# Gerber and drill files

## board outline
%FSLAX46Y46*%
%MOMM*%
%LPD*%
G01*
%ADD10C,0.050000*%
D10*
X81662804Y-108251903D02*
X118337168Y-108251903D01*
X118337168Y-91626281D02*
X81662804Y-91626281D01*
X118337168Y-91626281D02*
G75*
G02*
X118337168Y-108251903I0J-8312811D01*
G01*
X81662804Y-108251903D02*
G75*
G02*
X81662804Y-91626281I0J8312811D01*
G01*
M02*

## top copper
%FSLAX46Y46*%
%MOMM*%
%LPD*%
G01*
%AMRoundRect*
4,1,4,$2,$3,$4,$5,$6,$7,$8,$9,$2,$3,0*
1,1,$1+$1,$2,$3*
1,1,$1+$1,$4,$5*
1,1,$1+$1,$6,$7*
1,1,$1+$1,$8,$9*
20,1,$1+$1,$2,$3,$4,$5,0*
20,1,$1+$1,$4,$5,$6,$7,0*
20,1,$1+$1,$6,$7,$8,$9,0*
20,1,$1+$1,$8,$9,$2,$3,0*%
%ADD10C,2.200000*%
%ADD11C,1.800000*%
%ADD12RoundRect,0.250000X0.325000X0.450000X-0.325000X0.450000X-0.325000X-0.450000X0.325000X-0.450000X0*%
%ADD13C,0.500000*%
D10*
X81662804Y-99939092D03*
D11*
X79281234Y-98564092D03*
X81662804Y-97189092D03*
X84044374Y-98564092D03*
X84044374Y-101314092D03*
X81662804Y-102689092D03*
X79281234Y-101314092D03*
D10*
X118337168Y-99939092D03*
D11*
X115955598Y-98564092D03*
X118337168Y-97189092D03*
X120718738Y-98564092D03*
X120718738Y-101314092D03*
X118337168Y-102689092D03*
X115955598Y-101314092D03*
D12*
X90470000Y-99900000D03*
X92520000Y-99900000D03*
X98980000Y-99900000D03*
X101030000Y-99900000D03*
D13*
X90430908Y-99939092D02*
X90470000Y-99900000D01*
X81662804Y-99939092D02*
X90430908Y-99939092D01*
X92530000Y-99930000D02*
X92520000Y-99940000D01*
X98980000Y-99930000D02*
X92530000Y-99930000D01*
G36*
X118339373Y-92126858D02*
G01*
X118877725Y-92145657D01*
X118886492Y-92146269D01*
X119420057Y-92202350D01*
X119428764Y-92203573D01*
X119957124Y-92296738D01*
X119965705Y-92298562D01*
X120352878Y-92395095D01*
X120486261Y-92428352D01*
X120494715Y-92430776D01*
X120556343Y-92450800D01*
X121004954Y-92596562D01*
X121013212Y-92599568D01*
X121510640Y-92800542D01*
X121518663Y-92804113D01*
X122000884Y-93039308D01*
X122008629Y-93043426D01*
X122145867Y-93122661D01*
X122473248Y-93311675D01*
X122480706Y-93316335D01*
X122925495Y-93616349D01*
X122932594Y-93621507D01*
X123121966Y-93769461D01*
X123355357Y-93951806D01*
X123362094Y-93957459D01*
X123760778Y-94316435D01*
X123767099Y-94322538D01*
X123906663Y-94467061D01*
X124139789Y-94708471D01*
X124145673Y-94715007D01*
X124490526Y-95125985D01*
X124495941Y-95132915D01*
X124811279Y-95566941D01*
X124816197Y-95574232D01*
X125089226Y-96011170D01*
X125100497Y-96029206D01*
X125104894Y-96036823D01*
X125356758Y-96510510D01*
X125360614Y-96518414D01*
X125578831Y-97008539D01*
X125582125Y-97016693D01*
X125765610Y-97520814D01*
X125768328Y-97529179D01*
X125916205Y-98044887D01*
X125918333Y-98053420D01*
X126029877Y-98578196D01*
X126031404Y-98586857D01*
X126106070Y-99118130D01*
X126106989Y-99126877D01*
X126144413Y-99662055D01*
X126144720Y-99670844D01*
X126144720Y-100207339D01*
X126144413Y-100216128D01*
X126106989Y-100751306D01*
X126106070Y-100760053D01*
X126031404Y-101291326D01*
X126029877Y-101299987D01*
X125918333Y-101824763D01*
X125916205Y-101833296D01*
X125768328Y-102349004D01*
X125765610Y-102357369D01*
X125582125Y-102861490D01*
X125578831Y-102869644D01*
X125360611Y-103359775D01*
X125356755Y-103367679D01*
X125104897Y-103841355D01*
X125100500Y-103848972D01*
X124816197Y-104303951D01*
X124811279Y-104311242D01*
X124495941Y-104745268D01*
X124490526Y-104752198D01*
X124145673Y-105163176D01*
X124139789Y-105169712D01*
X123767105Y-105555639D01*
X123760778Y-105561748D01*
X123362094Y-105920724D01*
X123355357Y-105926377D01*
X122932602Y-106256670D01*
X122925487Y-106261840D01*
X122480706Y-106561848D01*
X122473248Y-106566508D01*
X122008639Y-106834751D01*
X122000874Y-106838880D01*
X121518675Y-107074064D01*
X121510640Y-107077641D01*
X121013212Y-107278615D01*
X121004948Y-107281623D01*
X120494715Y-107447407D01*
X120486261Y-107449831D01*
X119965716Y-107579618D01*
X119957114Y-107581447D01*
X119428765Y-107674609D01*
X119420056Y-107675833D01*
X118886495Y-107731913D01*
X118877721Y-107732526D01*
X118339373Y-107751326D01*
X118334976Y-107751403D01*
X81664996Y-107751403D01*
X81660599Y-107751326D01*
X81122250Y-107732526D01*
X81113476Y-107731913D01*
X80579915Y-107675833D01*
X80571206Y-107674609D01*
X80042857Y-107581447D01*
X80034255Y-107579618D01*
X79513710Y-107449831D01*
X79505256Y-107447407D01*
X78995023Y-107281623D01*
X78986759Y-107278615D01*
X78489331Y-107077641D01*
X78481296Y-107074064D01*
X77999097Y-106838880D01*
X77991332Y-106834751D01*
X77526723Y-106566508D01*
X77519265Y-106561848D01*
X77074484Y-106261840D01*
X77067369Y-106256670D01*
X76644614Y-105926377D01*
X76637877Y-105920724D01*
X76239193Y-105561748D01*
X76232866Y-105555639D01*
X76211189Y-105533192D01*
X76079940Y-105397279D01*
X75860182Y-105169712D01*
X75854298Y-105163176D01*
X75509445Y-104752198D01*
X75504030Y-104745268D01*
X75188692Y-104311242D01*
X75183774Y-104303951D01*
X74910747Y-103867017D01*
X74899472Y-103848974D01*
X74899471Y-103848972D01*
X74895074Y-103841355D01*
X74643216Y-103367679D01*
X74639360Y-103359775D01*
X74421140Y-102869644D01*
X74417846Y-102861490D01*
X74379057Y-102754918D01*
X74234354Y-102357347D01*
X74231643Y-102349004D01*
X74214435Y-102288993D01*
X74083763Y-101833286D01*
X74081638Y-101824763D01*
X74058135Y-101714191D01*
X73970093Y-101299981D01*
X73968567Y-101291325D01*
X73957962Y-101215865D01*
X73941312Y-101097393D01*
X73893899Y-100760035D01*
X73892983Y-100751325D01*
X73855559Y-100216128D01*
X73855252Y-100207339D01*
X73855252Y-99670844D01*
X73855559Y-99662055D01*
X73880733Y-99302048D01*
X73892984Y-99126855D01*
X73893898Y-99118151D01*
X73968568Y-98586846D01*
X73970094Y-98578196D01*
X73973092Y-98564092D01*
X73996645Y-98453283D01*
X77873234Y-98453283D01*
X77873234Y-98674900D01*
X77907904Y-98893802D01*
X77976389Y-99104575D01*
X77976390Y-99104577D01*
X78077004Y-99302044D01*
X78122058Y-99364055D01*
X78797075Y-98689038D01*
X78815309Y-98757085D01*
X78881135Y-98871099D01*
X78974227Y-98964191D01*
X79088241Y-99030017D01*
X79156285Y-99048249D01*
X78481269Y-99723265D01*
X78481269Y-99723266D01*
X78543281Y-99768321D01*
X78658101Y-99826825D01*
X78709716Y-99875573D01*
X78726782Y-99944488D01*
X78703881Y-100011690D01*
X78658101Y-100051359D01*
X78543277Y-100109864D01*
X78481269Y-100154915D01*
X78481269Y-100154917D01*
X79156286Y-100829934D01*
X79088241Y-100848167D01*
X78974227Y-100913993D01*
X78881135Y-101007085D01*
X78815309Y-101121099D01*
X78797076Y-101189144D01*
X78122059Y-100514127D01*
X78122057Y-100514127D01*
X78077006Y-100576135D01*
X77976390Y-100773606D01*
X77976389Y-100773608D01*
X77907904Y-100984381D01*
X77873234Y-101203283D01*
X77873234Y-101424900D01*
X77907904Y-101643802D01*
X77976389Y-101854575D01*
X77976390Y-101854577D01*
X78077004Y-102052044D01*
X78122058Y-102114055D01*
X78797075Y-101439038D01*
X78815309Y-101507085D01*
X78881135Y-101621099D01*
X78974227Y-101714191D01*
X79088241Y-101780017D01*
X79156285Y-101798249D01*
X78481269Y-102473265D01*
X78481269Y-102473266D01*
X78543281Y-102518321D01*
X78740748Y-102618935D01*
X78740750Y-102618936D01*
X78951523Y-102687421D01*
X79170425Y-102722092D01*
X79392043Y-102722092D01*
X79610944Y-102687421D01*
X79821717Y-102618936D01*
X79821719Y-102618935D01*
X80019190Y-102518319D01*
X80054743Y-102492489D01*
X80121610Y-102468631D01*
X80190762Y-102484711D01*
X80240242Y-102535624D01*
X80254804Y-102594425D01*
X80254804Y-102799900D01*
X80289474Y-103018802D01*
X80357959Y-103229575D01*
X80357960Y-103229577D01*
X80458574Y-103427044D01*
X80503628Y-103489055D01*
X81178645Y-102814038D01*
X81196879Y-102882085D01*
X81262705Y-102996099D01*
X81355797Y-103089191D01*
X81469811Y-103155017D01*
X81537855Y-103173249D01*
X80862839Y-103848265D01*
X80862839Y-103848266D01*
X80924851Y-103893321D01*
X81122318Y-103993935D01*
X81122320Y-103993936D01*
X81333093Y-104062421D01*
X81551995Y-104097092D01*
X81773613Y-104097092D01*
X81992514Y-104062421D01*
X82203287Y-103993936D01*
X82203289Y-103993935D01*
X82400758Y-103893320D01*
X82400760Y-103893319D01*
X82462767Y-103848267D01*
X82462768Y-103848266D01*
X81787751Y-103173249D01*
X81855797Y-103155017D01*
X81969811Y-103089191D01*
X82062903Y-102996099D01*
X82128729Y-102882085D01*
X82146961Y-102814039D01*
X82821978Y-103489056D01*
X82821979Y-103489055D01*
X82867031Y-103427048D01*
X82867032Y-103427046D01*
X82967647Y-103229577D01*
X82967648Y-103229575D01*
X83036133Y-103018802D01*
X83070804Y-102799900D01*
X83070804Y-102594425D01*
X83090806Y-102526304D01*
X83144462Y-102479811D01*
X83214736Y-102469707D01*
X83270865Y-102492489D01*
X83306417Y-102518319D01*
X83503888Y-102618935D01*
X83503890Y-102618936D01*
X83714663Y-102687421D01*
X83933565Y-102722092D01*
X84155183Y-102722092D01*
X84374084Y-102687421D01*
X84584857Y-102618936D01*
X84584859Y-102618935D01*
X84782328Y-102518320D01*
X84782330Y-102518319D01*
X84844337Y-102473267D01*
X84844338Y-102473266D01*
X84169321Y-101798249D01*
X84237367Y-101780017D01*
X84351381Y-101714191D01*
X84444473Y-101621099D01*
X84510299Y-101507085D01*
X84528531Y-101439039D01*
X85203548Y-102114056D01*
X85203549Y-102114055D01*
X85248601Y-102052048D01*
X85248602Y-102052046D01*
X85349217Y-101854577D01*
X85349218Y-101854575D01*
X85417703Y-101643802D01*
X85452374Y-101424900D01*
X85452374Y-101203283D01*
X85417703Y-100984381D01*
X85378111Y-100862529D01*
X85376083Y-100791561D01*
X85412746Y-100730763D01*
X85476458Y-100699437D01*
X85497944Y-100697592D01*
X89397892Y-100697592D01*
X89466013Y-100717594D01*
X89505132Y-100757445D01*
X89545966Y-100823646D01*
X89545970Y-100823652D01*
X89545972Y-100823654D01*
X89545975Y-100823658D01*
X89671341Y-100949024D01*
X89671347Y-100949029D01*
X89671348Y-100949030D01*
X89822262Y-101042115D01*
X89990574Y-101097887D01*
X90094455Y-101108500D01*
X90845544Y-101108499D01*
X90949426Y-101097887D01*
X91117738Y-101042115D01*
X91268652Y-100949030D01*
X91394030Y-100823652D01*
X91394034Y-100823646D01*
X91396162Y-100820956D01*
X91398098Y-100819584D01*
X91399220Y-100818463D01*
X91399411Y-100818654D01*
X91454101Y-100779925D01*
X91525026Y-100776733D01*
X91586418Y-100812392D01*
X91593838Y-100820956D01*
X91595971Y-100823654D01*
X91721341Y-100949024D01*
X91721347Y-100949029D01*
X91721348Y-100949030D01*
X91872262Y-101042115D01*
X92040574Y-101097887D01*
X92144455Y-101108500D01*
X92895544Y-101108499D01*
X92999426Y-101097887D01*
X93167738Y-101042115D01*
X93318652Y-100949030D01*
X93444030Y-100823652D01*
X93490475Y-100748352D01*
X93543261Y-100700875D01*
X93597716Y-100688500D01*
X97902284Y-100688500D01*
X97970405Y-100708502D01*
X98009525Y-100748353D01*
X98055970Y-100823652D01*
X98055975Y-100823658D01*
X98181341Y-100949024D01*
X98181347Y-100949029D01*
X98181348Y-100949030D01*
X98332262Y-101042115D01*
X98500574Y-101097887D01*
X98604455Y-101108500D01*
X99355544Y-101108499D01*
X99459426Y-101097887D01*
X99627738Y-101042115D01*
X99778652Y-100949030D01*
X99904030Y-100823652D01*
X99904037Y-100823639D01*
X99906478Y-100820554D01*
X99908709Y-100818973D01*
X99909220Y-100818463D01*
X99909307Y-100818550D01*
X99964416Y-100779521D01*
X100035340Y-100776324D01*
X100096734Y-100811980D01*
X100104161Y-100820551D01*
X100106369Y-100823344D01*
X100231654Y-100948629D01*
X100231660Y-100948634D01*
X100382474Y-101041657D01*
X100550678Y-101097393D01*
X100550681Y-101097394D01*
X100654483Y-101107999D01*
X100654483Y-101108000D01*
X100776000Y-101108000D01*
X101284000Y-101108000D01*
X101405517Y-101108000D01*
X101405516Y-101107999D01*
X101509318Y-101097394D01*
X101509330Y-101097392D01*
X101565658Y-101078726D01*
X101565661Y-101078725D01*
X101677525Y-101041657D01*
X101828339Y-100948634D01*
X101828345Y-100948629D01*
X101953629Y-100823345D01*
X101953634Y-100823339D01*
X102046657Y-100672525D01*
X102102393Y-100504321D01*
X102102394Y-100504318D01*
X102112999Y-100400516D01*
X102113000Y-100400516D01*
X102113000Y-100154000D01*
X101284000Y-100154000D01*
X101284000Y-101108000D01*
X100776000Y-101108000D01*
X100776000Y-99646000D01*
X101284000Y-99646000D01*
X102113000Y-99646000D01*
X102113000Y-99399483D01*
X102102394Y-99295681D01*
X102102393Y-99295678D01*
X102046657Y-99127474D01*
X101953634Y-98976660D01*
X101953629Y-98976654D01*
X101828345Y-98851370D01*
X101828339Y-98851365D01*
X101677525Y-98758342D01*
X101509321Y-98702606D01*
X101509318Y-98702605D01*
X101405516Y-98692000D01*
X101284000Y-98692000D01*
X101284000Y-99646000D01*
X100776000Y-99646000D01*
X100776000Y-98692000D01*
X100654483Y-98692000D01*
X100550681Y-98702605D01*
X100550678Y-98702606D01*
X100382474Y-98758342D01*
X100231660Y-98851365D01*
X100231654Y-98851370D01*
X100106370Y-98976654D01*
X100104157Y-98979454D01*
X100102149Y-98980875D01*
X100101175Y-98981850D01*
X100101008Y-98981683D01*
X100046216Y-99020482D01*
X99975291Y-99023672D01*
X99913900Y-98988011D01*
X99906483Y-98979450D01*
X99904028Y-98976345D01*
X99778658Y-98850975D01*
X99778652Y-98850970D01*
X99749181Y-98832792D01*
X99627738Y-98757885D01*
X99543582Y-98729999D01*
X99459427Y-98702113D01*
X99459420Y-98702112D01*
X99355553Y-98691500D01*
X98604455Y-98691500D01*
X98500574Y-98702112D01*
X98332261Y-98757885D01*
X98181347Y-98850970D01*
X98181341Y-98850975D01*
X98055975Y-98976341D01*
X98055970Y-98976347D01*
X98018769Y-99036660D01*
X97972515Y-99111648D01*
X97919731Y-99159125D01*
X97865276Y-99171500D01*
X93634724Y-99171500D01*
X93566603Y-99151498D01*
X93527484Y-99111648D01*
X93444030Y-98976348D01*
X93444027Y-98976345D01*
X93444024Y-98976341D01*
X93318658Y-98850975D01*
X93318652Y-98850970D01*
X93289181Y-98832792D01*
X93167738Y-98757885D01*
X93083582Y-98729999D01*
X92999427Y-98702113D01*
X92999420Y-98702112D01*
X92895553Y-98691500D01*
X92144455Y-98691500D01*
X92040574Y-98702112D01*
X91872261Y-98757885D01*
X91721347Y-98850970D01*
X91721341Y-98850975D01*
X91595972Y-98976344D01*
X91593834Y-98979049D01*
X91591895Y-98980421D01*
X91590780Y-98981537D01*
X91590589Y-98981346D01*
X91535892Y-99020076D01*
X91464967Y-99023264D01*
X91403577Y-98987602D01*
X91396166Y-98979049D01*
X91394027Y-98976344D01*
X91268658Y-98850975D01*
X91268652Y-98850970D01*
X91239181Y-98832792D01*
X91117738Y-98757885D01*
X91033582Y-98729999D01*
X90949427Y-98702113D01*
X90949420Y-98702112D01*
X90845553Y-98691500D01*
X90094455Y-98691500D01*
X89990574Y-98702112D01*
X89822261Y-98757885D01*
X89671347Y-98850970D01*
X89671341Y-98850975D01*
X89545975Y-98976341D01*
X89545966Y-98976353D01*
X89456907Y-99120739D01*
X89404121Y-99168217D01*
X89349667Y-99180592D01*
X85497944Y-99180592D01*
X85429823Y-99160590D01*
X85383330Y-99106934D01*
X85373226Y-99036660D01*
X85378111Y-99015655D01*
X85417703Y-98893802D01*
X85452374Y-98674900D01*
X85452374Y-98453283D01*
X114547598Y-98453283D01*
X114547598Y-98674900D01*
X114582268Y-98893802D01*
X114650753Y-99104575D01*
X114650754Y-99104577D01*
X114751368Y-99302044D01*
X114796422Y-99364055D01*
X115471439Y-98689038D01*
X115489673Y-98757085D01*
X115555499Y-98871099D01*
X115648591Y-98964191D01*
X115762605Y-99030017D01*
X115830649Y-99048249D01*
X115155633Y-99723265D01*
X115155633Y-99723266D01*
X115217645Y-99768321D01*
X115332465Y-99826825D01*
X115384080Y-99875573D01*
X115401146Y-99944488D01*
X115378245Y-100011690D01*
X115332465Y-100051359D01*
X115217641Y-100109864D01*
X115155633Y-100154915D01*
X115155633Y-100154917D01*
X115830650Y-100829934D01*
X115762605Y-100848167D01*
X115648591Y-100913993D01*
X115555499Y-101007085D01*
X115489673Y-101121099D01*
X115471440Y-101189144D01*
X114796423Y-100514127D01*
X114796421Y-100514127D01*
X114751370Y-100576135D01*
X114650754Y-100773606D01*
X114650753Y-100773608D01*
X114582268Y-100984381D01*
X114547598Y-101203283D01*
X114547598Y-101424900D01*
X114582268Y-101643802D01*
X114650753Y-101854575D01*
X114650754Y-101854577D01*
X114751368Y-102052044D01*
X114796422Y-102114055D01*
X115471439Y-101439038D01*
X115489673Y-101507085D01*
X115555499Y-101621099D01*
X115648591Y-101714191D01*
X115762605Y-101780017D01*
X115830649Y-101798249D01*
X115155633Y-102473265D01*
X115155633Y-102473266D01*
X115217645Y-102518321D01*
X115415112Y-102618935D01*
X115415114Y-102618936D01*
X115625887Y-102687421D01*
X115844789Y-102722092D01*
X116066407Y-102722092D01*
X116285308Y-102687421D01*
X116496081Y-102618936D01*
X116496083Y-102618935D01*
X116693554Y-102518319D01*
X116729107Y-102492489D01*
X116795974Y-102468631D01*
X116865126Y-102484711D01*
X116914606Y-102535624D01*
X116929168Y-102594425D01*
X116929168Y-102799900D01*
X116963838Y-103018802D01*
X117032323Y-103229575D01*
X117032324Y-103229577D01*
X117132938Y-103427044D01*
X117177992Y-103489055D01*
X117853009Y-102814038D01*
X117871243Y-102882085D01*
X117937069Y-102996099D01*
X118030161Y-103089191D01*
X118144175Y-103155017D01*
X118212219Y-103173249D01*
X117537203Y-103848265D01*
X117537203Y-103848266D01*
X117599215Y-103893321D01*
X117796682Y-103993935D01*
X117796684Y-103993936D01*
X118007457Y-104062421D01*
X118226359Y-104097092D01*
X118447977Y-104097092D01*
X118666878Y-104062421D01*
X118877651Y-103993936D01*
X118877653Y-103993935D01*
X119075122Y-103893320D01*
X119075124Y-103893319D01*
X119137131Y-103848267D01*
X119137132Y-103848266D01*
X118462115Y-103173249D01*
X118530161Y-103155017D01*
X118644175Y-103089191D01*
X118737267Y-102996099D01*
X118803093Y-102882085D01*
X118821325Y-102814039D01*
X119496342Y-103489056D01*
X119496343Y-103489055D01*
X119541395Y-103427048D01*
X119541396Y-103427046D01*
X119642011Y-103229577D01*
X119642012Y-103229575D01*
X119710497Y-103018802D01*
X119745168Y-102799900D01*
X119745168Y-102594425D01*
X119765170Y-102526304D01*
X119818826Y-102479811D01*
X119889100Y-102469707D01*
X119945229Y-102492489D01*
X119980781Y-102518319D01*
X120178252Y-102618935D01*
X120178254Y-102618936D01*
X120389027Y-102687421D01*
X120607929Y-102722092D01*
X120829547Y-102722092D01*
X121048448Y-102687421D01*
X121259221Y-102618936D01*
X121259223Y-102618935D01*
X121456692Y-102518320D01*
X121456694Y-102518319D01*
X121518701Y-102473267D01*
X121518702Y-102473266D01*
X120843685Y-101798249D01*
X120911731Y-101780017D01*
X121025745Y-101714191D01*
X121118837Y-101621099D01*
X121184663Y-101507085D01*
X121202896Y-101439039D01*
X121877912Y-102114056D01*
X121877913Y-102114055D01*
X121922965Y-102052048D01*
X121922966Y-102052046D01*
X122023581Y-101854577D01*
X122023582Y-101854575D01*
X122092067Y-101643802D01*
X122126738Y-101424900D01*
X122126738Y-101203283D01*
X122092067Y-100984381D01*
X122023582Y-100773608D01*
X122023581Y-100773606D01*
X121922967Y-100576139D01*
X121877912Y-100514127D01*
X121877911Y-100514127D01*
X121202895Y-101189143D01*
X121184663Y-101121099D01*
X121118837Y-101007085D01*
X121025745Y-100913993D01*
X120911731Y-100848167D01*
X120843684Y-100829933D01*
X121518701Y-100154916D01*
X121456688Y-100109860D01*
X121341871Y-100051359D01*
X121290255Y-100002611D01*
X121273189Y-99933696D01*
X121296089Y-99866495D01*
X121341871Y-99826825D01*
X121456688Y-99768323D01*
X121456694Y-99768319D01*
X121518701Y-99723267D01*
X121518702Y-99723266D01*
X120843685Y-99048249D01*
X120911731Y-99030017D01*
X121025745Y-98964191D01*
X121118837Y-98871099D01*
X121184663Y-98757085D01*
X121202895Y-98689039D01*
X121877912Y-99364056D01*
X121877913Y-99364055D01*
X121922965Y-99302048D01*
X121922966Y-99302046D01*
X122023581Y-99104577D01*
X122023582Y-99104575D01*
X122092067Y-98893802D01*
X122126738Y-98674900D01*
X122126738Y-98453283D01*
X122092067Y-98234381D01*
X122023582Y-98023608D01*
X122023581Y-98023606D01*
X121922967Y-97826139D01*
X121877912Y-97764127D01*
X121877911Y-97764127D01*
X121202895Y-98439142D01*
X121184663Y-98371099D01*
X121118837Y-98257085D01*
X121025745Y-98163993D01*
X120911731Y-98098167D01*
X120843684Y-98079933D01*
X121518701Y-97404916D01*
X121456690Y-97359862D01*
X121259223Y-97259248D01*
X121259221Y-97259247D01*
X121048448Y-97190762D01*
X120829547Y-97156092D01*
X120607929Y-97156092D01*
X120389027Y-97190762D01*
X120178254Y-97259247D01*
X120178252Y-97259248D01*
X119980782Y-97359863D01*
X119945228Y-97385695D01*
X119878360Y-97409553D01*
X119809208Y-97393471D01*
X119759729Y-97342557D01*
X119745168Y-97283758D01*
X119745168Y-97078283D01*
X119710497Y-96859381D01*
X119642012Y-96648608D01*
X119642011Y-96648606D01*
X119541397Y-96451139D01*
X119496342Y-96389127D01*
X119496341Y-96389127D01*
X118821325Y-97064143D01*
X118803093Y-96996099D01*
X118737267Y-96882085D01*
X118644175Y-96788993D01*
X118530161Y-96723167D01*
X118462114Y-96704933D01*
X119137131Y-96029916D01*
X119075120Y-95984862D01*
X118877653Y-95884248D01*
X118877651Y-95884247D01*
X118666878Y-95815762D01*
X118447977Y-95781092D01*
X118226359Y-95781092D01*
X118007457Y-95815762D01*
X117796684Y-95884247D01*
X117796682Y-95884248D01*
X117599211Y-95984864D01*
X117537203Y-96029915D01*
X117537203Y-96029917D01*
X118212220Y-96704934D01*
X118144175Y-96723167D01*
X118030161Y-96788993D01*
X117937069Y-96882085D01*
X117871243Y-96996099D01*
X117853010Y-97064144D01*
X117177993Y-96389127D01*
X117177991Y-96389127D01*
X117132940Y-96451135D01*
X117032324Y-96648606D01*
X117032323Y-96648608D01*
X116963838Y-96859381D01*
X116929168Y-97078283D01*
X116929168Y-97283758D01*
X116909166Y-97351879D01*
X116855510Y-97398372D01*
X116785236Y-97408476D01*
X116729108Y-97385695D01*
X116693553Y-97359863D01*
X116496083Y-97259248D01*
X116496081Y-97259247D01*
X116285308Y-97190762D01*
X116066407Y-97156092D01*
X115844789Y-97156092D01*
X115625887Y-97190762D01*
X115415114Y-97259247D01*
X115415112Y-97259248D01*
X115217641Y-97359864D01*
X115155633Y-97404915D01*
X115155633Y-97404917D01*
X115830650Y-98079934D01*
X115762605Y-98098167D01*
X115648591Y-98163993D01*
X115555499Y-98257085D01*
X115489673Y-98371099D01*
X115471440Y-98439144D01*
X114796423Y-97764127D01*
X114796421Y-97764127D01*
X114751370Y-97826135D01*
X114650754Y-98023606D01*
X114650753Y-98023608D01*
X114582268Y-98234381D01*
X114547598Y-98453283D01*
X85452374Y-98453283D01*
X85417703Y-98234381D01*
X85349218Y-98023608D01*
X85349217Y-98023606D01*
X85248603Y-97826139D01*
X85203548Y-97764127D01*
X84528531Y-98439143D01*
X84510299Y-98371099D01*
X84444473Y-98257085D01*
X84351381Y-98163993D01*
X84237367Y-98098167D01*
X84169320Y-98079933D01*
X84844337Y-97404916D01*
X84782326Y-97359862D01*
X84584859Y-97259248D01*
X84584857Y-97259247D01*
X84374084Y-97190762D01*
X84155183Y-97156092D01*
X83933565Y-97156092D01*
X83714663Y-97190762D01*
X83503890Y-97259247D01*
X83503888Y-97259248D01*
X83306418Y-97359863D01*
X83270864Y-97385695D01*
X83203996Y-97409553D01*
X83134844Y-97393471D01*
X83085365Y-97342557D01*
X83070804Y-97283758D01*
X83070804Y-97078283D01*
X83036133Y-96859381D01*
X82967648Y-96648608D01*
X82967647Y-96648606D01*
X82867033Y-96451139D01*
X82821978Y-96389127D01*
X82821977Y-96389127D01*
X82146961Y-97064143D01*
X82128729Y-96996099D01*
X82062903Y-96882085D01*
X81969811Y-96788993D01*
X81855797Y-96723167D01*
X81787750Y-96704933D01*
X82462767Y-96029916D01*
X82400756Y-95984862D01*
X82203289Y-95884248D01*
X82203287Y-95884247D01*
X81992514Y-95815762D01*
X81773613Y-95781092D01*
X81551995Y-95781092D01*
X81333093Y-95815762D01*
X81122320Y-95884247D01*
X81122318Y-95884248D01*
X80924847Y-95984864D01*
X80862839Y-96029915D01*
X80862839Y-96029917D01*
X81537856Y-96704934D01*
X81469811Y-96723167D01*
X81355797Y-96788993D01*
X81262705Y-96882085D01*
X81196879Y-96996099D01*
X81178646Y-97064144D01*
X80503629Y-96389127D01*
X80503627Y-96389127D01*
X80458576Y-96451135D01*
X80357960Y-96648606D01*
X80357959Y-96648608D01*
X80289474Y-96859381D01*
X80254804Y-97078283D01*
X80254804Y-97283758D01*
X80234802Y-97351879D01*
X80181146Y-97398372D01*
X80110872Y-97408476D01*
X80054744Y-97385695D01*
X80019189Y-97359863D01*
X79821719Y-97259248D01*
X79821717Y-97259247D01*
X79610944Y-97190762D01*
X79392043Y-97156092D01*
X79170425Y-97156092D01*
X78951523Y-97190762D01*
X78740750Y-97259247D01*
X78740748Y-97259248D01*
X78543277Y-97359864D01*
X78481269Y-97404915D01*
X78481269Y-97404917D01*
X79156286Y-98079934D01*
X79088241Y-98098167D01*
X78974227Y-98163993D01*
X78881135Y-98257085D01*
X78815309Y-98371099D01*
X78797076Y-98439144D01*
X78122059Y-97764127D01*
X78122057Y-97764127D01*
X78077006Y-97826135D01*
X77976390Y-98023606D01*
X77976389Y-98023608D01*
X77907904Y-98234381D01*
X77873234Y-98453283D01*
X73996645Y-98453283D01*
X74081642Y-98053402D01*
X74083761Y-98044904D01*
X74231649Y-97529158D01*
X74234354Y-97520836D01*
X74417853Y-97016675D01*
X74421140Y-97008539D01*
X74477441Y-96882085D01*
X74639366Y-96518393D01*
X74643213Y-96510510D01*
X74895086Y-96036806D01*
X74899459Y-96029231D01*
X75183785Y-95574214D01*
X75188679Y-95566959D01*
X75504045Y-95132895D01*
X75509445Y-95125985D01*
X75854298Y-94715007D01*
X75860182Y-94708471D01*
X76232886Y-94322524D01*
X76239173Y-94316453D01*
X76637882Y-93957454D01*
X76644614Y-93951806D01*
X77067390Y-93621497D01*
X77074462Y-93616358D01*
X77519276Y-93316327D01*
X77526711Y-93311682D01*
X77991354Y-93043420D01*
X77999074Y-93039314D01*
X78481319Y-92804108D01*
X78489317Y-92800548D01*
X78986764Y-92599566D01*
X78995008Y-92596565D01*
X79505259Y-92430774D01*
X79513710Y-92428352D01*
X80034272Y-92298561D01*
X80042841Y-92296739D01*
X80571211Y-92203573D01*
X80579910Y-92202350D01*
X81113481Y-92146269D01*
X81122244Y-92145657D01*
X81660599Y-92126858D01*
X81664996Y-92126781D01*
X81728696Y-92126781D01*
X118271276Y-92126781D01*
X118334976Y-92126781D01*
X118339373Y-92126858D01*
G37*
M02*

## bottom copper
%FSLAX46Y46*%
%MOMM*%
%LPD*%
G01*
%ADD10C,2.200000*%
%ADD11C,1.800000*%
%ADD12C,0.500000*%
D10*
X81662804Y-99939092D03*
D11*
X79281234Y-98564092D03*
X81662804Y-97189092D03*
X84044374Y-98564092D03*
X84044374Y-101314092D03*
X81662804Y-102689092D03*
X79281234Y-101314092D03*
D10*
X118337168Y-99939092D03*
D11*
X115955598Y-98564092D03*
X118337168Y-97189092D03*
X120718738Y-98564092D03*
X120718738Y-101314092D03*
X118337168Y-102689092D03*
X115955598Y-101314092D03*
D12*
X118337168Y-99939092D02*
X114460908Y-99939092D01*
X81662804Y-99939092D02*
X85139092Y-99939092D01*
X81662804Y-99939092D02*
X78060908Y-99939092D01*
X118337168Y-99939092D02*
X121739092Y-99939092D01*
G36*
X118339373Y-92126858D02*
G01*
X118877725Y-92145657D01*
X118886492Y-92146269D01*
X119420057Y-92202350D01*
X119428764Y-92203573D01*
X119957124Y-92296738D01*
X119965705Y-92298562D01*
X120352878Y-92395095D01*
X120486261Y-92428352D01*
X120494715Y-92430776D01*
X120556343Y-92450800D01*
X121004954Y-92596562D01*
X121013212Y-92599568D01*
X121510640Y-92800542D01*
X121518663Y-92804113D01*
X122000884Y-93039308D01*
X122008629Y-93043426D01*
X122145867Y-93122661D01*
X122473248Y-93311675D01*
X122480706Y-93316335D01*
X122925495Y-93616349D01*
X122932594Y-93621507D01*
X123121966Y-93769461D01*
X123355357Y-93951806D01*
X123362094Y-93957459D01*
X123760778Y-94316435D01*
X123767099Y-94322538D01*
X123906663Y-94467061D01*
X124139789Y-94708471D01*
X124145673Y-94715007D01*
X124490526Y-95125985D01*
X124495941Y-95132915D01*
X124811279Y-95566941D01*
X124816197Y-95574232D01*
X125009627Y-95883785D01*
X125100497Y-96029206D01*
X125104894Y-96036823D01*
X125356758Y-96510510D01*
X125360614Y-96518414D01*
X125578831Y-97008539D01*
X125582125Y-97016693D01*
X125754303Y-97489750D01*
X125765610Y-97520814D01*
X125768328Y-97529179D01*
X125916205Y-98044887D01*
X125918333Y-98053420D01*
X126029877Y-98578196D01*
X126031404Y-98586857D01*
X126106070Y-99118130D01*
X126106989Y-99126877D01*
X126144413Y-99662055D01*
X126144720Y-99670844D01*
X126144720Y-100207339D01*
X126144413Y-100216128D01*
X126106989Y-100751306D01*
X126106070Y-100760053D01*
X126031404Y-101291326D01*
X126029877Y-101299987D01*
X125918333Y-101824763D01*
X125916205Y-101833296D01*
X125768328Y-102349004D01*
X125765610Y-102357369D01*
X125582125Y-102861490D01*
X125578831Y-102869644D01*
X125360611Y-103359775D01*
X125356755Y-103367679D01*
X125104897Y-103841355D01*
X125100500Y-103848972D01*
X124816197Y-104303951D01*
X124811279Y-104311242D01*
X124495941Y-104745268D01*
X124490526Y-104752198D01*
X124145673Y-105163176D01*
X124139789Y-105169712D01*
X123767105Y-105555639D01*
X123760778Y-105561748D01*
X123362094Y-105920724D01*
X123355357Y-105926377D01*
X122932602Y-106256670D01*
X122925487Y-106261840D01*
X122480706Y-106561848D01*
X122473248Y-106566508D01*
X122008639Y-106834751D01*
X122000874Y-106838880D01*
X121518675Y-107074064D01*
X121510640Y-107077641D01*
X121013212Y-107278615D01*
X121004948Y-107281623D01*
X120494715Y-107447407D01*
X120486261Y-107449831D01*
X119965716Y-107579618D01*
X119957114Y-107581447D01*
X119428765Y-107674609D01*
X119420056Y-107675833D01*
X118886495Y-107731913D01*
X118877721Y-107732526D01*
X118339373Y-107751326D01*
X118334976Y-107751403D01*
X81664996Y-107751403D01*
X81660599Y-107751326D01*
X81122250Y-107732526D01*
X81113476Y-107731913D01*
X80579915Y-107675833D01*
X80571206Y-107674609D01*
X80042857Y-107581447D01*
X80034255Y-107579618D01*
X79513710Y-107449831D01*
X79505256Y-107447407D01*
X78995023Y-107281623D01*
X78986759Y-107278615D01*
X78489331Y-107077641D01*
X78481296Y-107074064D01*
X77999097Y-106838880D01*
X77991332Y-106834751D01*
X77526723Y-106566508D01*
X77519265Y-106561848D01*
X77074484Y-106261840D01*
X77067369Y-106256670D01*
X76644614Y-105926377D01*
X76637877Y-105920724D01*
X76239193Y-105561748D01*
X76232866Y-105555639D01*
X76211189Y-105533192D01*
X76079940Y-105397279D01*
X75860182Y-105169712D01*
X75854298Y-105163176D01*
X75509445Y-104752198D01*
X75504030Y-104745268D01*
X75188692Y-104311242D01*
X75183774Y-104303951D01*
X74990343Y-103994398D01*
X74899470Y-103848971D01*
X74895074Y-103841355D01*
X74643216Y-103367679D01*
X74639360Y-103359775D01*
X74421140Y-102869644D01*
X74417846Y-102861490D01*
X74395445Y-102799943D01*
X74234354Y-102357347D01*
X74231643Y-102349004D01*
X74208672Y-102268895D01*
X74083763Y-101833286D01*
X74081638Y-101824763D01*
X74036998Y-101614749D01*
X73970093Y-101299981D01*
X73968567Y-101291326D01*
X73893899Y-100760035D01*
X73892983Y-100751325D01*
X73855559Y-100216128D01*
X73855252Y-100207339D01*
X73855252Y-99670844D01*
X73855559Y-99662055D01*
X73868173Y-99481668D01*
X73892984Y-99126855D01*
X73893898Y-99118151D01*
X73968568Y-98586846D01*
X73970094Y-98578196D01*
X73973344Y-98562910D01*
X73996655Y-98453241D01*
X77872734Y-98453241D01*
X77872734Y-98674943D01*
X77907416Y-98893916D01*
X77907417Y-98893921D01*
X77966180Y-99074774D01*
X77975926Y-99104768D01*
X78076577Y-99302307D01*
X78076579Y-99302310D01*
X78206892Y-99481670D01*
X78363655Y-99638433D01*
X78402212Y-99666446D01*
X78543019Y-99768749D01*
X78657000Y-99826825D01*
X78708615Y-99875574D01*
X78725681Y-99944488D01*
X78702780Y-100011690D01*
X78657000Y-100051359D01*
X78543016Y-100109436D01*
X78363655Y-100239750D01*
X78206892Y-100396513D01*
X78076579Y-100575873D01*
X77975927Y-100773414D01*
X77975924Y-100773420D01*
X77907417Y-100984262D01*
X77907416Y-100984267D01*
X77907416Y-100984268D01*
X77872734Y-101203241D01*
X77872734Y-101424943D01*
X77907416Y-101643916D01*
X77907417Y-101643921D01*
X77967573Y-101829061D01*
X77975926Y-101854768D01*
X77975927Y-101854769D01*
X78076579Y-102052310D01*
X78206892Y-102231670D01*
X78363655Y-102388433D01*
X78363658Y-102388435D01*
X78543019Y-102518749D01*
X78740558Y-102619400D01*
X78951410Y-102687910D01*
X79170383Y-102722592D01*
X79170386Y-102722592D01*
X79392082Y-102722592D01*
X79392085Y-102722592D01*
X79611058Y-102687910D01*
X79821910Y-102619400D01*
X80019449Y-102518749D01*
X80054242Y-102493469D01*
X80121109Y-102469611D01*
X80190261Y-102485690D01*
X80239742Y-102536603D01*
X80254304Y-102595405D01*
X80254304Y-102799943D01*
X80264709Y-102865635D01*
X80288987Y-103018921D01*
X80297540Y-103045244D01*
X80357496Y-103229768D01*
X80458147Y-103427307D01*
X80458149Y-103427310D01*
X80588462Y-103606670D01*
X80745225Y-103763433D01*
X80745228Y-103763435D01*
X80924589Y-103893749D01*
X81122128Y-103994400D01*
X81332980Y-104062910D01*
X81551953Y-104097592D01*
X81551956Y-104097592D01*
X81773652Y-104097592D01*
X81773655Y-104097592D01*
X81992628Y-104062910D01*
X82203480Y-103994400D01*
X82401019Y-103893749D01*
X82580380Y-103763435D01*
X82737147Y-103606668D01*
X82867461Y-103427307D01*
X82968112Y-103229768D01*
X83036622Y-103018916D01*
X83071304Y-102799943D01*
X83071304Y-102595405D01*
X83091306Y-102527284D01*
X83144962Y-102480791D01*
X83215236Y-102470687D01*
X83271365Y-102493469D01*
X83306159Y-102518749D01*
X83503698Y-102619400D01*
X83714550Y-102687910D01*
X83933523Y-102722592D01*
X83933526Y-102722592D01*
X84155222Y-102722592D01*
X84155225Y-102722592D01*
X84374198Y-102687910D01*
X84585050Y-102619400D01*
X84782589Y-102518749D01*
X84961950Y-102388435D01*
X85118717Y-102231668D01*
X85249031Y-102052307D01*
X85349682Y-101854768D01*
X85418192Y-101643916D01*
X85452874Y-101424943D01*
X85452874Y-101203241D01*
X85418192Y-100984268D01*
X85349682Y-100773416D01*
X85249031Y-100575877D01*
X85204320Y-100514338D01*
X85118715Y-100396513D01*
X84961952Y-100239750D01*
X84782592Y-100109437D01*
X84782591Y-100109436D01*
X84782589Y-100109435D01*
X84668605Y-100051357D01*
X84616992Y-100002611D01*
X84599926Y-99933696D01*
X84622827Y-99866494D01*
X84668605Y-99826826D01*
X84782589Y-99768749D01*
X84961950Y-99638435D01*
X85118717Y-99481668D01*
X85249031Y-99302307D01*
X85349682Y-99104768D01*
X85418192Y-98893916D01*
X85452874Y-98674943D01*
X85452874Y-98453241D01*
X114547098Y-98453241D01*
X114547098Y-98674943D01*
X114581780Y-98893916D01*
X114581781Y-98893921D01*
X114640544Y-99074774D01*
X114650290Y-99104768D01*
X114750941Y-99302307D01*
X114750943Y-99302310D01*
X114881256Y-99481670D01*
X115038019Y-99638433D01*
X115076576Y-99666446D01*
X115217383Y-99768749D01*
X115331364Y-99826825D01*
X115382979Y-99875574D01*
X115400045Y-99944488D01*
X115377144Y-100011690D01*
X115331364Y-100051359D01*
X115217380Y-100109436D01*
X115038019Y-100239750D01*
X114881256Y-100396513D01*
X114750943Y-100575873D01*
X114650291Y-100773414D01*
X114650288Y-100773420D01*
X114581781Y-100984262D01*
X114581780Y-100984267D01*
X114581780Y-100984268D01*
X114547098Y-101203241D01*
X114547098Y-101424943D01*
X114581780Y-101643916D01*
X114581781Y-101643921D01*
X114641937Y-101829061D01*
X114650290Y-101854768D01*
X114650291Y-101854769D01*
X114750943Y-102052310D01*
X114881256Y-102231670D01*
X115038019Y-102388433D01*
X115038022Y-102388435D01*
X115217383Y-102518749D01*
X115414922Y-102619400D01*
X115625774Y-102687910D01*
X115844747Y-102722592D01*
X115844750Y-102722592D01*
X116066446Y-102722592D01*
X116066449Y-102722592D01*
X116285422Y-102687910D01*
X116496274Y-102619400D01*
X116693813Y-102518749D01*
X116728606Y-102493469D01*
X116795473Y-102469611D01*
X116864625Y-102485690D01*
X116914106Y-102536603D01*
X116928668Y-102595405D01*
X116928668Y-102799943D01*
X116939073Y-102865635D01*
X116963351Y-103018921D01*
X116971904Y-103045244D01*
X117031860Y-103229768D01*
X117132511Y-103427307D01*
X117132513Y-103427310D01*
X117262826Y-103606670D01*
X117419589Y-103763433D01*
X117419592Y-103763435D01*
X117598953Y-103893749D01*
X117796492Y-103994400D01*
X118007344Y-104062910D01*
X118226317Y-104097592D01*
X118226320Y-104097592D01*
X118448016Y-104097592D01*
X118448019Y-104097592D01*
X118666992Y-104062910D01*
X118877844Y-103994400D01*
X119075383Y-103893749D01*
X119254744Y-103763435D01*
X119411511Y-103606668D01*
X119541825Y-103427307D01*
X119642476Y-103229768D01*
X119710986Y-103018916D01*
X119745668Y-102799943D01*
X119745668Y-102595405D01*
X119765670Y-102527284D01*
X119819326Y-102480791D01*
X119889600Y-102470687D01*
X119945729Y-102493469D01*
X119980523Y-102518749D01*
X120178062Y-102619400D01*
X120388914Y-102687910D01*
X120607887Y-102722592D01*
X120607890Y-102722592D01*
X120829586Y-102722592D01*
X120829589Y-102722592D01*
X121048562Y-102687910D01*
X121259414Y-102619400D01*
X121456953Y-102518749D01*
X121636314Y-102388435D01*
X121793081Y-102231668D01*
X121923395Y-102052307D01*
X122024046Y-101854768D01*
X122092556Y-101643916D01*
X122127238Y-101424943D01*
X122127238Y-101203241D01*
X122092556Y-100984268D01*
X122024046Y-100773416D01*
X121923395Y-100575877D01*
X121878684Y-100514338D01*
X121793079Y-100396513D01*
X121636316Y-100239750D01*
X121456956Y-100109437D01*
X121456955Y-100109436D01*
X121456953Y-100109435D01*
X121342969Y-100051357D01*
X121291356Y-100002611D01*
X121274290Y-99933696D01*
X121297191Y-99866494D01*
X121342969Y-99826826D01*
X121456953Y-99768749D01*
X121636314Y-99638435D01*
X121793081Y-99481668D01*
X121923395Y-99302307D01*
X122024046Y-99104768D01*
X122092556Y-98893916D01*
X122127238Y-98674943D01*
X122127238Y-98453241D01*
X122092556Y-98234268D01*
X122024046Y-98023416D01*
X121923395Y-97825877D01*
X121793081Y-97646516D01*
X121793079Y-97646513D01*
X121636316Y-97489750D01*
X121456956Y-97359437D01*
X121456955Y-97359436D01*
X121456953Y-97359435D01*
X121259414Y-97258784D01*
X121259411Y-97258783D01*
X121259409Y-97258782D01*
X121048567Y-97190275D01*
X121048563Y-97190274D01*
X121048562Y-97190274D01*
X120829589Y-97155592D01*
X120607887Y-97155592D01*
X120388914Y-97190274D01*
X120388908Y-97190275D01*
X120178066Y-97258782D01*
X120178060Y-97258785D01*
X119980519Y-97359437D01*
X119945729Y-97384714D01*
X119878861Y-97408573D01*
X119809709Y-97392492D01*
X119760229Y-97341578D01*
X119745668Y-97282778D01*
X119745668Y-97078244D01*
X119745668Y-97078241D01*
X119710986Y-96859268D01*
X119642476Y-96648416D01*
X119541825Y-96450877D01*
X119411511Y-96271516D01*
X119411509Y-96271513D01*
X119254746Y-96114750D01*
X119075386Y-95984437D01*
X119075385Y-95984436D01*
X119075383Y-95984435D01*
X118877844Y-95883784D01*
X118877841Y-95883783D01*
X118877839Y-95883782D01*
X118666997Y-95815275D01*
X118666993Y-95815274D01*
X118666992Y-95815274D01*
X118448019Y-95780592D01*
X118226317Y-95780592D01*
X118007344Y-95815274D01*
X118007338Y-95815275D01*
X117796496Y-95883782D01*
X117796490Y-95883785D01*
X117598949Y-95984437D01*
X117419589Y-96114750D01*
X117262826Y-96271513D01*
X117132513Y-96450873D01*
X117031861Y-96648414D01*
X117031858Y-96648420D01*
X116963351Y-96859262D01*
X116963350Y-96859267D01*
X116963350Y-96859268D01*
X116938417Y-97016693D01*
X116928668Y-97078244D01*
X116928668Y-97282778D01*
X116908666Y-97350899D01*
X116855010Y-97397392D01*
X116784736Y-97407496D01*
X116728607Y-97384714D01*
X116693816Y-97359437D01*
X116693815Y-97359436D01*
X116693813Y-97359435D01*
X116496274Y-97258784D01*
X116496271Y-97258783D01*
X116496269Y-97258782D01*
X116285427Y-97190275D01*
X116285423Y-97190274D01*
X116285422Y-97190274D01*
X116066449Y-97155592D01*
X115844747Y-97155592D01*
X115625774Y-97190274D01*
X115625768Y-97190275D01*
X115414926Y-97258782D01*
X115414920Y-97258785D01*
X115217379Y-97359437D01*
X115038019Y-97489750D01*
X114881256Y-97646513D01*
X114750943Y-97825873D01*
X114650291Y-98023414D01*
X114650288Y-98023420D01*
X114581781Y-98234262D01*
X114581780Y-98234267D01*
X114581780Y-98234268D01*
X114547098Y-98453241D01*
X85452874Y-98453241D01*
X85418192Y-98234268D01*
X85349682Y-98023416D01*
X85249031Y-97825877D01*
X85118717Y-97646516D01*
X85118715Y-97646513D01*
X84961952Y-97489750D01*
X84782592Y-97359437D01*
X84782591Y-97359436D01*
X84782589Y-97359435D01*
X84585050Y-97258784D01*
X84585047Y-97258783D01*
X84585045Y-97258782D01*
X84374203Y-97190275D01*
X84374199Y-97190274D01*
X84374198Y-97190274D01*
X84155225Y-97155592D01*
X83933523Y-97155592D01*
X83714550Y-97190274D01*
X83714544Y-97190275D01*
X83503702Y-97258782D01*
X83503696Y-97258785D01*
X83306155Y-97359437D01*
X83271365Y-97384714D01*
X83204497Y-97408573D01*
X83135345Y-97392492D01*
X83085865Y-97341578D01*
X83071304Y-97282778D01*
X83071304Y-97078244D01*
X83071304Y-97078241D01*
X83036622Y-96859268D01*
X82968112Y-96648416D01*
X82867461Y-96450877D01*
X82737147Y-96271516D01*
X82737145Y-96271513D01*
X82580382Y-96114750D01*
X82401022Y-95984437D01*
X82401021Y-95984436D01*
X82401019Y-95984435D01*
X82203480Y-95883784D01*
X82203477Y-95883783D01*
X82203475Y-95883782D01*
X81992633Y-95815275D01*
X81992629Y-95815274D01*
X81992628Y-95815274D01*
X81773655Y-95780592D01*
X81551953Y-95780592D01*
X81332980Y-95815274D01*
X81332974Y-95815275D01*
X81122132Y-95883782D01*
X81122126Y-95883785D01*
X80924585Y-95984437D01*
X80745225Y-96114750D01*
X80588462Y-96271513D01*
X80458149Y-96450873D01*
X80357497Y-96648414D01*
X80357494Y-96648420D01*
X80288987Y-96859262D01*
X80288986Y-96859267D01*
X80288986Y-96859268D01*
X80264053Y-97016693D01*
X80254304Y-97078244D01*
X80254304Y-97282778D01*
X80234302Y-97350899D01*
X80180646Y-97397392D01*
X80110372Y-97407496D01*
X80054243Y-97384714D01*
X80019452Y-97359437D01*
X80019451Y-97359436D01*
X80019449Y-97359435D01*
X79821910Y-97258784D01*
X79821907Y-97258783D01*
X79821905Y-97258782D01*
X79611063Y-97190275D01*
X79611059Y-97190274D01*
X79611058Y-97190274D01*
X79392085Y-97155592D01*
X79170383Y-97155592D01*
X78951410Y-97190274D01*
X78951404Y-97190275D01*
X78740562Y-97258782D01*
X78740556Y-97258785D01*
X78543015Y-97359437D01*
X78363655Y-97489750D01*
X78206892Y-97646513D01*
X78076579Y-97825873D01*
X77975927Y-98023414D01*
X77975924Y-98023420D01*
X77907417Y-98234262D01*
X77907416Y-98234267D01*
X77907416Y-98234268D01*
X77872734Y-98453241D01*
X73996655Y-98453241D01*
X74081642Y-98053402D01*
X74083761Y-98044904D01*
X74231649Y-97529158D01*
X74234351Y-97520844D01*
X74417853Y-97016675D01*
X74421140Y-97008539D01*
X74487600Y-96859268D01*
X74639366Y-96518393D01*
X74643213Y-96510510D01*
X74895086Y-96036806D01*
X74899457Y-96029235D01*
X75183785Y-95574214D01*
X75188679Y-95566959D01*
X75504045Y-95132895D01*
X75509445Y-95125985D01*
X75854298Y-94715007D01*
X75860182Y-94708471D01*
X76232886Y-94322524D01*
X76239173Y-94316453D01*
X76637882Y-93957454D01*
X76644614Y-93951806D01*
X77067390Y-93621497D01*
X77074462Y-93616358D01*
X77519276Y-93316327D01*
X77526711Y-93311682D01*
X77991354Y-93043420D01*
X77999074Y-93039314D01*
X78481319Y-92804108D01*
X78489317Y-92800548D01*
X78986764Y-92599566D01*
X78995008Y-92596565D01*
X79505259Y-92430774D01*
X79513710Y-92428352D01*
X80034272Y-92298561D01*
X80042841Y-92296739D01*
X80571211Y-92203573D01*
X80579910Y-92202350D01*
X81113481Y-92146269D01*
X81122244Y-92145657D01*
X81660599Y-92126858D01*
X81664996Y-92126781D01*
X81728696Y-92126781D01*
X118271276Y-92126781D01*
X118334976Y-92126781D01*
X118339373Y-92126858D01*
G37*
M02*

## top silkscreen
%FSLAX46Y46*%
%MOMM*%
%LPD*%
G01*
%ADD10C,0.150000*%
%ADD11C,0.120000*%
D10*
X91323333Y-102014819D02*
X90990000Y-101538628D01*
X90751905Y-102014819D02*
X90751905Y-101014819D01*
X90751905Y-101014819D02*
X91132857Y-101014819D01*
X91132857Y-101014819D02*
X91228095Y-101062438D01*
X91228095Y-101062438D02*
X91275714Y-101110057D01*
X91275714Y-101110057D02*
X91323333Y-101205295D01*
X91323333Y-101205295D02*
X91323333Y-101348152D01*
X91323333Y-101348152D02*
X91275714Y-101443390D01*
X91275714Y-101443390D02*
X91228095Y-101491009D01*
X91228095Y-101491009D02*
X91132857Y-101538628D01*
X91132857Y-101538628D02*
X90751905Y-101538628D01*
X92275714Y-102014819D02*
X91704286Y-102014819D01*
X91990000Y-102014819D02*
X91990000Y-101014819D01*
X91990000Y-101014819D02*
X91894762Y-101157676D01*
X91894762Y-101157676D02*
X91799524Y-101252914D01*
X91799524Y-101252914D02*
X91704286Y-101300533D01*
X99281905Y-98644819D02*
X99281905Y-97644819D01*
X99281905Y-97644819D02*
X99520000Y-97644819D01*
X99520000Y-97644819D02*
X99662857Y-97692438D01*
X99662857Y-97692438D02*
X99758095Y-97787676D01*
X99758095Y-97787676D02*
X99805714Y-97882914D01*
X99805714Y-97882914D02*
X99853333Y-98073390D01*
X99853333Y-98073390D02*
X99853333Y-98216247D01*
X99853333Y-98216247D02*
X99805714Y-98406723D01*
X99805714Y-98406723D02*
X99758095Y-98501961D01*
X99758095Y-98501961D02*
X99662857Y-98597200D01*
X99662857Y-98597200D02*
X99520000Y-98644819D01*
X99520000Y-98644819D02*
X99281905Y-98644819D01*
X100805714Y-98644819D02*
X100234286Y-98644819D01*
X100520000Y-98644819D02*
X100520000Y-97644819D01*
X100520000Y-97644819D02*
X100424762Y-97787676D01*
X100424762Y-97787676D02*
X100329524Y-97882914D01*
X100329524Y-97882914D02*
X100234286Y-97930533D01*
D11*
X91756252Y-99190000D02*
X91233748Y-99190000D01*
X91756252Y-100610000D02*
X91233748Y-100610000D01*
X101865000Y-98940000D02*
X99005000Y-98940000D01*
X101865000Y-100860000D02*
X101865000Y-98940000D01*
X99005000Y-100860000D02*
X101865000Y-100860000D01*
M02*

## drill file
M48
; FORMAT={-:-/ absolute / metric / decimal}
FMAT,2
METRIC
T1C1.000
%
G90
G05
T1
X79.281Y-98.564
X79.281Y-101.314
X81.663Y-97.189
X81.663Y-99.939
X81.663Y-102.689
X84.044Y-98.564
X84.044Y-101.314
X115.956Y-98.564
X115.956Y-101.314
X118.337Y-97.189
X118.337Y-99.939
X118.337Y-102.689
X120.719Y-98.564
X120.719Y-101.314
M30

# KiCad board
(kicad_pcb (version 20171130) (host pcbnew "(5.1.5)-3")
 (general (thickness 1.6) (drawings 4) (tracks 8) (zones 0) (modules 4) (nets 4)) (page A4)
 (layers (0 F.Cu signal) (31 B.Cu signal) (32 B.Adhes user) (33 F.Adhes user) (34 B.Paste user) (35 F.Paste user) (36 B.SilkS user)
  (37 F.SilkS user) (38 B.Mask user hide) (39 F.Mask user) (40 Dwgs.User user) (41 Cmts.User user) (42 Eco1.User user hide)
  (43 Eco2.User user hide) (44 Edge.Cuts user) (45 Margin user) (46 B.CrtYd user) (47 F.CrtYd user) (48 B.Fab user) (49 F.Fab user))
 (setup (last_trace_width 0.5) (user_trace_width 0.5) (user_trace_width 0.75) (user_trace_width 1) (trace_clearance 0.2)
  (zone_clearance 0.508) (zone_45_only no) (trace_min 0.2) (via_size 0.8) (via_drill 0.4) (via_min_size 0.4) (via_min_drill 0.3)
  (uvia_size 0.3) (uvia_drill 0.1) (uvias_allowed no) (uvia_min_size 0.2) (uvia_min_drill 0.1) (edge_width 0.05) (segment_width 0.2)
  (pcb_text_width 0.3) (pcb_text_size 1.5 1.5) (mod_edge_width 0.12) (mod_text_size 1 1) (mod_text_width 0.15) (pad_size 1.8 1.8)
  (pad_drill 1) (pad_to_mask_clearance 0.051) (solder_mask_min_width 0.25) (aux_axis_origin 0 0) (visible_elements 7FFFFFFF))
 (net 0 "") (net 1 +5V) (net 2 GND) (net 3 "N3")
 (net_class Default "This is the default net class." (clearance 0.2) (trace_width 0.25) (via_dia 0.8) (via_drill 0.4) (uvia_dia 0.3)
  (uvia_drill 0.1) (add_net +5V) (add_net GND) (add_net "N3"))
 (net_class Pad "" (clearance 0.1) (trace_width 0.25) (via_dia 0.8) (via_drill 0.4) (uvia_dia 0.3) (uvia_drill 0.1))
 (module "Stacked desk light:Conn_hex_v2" (layer F.Cu) (at 81.662804 99.939092 90)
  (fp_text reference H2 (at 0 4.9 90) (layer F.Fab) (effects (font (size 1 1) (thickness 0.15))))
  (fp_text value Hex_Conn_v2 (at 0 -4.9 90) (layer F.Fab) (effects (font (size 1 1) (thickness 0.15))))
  (pad 7 thru_hole circle (at 0 0 90) (size 2.2 2.2) (drill 1) (layers *.Cu *.Mask) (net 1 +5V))
  (pad 1 thru_hole circle (at 1.375 -2.38157 90) (size 1.8 1.8) (drill 1) (layers *.Cu *.Mask) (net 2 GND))
  (pad 2 thru_hole circle (at 2.75 0 90) (size 1.8 1.8) (drill 1) (layers *.Cu *.Mask) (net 2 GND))
  (pad 3 thru_hole circle (at 1.375 2.38157 90) (size 1.8 1.8) (drill 1) (layers *.Cu *.Mask) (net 2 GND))
  (pad 4 thru_hole circle (at -1.375 2.38157 90) (size 1.8 1.8) (drill 1) (layers *.Cu *.Mask) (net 2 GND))
  (pad 5 thru_hole circle (at -2.75 0 90) (size 1.8 1.8) (drill 1) (layers *.Cu *.Mask) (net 2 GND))
  (pad 6 thru_hole circle (at -1.375 -2.38157 90) (size 1.8 1.8) (drill 1) (layers *.Cu *.Mask) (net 2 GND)))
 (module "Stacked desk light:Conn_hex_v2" (layer F.Cu) (at 118.337168 99.939092 90)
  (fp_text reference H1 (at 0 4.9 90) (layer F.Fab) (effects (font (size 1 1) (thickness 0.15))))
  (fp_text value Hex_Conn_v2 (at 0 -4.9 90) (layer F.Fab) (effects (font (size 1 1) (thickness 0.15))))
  (pad 7 thru_hole circle (at 0 0 90) (size 2.2 2.2) (drill 1) (layers *.Cu *.Mask) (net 1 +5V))
  (pad 1 thru_hole circle (at 1.375 -2.38157 90) (size 1.8 1.8) (drill 1) (layers *.Cu *.Mask) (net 2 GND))
  (pad 2 thru_hole circle (at 2.75 0 90) (size 1.8 1.8) (drill 1) (layers *.Cu *.Mask) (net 2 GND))
  (pad 3 thru_hole circle (at 1.375 2.38157 90) (size 1.8 1.8) (drill 1) (layers *.Cu *.Mask) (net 2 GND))
  (pad 4 thru_hole circle (at -1.375 2.38157 90) (size 1.8 1.8) (drill 1) (layers *.Cu *.Mask) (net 2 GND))
  (pad 5 thru_hole circle (at -2.75 0 90) (size 1.8 1.8) (drill 1) (layers *.Cu *.Mask) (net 2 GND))
  (pad 6 thru_hole circle (at -1.375 -2.38157 90) (size 1.8 1.8) (drill 1) (layers *.Cu *.Mask) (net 2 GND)))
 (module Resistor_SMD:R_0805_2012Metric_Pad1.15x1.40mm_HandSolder (layer F.Cu) (at 91.495 99.9 180)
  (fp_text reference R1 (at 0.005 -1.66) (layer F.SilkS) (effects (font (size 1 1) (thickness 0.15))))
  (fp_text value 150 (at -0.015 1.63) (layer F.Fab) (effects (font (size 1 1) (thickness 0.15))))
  (fp_line (start -0.261252 0.71) (end 0.261252 0.71) (layer F.SilkS) (width 0.12))
  (fp_line (start -0.261252 -0.71) (end 0.261252 -0.71) (layer F.SilkS) (width 0.12))
  (pad 2 smd roundrect (at 1.025 0 180) (size 1.15 1.4) (layers F.Cu F.Paste F.Mask) (roundrect_rratio 0.217391) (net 1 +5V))
  (pad 1 smd roundrect (at -1.025 0 180) (size 1.15 1.4) (layers F.Cu F.Paste F.Mask) (roundrect_rratio 0.217391) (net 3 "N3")))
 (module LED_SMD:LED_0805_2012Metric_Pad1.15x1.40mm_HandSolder (layer F.Cu) (at 100.005 99.9 180)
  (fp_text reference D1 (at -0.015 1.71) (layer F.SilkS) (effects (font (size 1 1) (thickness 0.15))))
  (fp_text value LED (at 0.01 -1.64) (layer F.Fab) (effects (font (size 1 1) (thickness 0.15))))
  (fp_line (start -1.86 0.96) (end 1 0.96) (layer F.SilkS) (width 0.12))
  (fp_line (start -1.86 -0.96) (end -1.86 0.96) (layer F.SilkS) (width 0.12))
  (fp_line (start 1 -0.96) (end -1.86 -0.96) (layer F.SilkS) (width 0.12))
  (pad 2 smd roundrect (at 1.025 0 180) (size 1.15 1.4) (layers F.Cu F.Paste F.Mask) (roundrect_rratio 0.217391) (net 3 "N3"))
  (pad 1 smd roundrect (at -1.025 0 180) (size 1.15 1.4) (layers F.Cu F.Paste F.Mask) (roundrect_rratio 0.217391) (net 2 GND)))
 (gr_line (start 81.662804 108.251903) (end 118.337168 108.251903) (layer Edge.Cuts) (width 0.05))
 (gr_line (start 118.337168 91.626281) (end 81.662804 91.626281) (layer Edge.Cuts) (width 0.05))
 (gr_arc (start 118.337168 99.939092) (end 118.337168 108.251903) (angle -180) (layer Edge.Cuts) (width 0.05))
 (gr_arc (start 81.662804 99.939092) (end 81.662804 91.626281) (angle -180) (layer Edge.Cuts) (width 0.05))
 (segment (start 90.430908 99.939092) (end 90.47 99.9) (width 0.5) (layer F.Cu) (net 1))
 (segment (start 81.662804 99.939092) (end 90.430908 99.939092) (width 0.5) (layer F.Cu) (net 1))
 (segment (start 118.337168 99.939092) (end 114.460908 99.939092) (width 0.5) (layer B.Cu) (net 1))
 (segment (start 81.662804 99.939092) (end 85.139092 99.939092) (width 0.5) (layer B.Cu) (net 1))
 (segment (start 81.662804 99.939092) (end 78.060908 99.939092) (width 0.5) (layer B.Cu) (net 1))
 (segment (start 118.337168 99.939092) (end 121.739092 99.939092) (width 0.5) (layer B.Cu) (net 1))
 (segment (start 92.53 99.93) (end 92.52 99.94) (width 0.5) (layer F.Cu) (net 3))
 (segment (start 98.98 99.93) (end 92.53 99.93) (width 0.5) (layer F.Cu) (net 3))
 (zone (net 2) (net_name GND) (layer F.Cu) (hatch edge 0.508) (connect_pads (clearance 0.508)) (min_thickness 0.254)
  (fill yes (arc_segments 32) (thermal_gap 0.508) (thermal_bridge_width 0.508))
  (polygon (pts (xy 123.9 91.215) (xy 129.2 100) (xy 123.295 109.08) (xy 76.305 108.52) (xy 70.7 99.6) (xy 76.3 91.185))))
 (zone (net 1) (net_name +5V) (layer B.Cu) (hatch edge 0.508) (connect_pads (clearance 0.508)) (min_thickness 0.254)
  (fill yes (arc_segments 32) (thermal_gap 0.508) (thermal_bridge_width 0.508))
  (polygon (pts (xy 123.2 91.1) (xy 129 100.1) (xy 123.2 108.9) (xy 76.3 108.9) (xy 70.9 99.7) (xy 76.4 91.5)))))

